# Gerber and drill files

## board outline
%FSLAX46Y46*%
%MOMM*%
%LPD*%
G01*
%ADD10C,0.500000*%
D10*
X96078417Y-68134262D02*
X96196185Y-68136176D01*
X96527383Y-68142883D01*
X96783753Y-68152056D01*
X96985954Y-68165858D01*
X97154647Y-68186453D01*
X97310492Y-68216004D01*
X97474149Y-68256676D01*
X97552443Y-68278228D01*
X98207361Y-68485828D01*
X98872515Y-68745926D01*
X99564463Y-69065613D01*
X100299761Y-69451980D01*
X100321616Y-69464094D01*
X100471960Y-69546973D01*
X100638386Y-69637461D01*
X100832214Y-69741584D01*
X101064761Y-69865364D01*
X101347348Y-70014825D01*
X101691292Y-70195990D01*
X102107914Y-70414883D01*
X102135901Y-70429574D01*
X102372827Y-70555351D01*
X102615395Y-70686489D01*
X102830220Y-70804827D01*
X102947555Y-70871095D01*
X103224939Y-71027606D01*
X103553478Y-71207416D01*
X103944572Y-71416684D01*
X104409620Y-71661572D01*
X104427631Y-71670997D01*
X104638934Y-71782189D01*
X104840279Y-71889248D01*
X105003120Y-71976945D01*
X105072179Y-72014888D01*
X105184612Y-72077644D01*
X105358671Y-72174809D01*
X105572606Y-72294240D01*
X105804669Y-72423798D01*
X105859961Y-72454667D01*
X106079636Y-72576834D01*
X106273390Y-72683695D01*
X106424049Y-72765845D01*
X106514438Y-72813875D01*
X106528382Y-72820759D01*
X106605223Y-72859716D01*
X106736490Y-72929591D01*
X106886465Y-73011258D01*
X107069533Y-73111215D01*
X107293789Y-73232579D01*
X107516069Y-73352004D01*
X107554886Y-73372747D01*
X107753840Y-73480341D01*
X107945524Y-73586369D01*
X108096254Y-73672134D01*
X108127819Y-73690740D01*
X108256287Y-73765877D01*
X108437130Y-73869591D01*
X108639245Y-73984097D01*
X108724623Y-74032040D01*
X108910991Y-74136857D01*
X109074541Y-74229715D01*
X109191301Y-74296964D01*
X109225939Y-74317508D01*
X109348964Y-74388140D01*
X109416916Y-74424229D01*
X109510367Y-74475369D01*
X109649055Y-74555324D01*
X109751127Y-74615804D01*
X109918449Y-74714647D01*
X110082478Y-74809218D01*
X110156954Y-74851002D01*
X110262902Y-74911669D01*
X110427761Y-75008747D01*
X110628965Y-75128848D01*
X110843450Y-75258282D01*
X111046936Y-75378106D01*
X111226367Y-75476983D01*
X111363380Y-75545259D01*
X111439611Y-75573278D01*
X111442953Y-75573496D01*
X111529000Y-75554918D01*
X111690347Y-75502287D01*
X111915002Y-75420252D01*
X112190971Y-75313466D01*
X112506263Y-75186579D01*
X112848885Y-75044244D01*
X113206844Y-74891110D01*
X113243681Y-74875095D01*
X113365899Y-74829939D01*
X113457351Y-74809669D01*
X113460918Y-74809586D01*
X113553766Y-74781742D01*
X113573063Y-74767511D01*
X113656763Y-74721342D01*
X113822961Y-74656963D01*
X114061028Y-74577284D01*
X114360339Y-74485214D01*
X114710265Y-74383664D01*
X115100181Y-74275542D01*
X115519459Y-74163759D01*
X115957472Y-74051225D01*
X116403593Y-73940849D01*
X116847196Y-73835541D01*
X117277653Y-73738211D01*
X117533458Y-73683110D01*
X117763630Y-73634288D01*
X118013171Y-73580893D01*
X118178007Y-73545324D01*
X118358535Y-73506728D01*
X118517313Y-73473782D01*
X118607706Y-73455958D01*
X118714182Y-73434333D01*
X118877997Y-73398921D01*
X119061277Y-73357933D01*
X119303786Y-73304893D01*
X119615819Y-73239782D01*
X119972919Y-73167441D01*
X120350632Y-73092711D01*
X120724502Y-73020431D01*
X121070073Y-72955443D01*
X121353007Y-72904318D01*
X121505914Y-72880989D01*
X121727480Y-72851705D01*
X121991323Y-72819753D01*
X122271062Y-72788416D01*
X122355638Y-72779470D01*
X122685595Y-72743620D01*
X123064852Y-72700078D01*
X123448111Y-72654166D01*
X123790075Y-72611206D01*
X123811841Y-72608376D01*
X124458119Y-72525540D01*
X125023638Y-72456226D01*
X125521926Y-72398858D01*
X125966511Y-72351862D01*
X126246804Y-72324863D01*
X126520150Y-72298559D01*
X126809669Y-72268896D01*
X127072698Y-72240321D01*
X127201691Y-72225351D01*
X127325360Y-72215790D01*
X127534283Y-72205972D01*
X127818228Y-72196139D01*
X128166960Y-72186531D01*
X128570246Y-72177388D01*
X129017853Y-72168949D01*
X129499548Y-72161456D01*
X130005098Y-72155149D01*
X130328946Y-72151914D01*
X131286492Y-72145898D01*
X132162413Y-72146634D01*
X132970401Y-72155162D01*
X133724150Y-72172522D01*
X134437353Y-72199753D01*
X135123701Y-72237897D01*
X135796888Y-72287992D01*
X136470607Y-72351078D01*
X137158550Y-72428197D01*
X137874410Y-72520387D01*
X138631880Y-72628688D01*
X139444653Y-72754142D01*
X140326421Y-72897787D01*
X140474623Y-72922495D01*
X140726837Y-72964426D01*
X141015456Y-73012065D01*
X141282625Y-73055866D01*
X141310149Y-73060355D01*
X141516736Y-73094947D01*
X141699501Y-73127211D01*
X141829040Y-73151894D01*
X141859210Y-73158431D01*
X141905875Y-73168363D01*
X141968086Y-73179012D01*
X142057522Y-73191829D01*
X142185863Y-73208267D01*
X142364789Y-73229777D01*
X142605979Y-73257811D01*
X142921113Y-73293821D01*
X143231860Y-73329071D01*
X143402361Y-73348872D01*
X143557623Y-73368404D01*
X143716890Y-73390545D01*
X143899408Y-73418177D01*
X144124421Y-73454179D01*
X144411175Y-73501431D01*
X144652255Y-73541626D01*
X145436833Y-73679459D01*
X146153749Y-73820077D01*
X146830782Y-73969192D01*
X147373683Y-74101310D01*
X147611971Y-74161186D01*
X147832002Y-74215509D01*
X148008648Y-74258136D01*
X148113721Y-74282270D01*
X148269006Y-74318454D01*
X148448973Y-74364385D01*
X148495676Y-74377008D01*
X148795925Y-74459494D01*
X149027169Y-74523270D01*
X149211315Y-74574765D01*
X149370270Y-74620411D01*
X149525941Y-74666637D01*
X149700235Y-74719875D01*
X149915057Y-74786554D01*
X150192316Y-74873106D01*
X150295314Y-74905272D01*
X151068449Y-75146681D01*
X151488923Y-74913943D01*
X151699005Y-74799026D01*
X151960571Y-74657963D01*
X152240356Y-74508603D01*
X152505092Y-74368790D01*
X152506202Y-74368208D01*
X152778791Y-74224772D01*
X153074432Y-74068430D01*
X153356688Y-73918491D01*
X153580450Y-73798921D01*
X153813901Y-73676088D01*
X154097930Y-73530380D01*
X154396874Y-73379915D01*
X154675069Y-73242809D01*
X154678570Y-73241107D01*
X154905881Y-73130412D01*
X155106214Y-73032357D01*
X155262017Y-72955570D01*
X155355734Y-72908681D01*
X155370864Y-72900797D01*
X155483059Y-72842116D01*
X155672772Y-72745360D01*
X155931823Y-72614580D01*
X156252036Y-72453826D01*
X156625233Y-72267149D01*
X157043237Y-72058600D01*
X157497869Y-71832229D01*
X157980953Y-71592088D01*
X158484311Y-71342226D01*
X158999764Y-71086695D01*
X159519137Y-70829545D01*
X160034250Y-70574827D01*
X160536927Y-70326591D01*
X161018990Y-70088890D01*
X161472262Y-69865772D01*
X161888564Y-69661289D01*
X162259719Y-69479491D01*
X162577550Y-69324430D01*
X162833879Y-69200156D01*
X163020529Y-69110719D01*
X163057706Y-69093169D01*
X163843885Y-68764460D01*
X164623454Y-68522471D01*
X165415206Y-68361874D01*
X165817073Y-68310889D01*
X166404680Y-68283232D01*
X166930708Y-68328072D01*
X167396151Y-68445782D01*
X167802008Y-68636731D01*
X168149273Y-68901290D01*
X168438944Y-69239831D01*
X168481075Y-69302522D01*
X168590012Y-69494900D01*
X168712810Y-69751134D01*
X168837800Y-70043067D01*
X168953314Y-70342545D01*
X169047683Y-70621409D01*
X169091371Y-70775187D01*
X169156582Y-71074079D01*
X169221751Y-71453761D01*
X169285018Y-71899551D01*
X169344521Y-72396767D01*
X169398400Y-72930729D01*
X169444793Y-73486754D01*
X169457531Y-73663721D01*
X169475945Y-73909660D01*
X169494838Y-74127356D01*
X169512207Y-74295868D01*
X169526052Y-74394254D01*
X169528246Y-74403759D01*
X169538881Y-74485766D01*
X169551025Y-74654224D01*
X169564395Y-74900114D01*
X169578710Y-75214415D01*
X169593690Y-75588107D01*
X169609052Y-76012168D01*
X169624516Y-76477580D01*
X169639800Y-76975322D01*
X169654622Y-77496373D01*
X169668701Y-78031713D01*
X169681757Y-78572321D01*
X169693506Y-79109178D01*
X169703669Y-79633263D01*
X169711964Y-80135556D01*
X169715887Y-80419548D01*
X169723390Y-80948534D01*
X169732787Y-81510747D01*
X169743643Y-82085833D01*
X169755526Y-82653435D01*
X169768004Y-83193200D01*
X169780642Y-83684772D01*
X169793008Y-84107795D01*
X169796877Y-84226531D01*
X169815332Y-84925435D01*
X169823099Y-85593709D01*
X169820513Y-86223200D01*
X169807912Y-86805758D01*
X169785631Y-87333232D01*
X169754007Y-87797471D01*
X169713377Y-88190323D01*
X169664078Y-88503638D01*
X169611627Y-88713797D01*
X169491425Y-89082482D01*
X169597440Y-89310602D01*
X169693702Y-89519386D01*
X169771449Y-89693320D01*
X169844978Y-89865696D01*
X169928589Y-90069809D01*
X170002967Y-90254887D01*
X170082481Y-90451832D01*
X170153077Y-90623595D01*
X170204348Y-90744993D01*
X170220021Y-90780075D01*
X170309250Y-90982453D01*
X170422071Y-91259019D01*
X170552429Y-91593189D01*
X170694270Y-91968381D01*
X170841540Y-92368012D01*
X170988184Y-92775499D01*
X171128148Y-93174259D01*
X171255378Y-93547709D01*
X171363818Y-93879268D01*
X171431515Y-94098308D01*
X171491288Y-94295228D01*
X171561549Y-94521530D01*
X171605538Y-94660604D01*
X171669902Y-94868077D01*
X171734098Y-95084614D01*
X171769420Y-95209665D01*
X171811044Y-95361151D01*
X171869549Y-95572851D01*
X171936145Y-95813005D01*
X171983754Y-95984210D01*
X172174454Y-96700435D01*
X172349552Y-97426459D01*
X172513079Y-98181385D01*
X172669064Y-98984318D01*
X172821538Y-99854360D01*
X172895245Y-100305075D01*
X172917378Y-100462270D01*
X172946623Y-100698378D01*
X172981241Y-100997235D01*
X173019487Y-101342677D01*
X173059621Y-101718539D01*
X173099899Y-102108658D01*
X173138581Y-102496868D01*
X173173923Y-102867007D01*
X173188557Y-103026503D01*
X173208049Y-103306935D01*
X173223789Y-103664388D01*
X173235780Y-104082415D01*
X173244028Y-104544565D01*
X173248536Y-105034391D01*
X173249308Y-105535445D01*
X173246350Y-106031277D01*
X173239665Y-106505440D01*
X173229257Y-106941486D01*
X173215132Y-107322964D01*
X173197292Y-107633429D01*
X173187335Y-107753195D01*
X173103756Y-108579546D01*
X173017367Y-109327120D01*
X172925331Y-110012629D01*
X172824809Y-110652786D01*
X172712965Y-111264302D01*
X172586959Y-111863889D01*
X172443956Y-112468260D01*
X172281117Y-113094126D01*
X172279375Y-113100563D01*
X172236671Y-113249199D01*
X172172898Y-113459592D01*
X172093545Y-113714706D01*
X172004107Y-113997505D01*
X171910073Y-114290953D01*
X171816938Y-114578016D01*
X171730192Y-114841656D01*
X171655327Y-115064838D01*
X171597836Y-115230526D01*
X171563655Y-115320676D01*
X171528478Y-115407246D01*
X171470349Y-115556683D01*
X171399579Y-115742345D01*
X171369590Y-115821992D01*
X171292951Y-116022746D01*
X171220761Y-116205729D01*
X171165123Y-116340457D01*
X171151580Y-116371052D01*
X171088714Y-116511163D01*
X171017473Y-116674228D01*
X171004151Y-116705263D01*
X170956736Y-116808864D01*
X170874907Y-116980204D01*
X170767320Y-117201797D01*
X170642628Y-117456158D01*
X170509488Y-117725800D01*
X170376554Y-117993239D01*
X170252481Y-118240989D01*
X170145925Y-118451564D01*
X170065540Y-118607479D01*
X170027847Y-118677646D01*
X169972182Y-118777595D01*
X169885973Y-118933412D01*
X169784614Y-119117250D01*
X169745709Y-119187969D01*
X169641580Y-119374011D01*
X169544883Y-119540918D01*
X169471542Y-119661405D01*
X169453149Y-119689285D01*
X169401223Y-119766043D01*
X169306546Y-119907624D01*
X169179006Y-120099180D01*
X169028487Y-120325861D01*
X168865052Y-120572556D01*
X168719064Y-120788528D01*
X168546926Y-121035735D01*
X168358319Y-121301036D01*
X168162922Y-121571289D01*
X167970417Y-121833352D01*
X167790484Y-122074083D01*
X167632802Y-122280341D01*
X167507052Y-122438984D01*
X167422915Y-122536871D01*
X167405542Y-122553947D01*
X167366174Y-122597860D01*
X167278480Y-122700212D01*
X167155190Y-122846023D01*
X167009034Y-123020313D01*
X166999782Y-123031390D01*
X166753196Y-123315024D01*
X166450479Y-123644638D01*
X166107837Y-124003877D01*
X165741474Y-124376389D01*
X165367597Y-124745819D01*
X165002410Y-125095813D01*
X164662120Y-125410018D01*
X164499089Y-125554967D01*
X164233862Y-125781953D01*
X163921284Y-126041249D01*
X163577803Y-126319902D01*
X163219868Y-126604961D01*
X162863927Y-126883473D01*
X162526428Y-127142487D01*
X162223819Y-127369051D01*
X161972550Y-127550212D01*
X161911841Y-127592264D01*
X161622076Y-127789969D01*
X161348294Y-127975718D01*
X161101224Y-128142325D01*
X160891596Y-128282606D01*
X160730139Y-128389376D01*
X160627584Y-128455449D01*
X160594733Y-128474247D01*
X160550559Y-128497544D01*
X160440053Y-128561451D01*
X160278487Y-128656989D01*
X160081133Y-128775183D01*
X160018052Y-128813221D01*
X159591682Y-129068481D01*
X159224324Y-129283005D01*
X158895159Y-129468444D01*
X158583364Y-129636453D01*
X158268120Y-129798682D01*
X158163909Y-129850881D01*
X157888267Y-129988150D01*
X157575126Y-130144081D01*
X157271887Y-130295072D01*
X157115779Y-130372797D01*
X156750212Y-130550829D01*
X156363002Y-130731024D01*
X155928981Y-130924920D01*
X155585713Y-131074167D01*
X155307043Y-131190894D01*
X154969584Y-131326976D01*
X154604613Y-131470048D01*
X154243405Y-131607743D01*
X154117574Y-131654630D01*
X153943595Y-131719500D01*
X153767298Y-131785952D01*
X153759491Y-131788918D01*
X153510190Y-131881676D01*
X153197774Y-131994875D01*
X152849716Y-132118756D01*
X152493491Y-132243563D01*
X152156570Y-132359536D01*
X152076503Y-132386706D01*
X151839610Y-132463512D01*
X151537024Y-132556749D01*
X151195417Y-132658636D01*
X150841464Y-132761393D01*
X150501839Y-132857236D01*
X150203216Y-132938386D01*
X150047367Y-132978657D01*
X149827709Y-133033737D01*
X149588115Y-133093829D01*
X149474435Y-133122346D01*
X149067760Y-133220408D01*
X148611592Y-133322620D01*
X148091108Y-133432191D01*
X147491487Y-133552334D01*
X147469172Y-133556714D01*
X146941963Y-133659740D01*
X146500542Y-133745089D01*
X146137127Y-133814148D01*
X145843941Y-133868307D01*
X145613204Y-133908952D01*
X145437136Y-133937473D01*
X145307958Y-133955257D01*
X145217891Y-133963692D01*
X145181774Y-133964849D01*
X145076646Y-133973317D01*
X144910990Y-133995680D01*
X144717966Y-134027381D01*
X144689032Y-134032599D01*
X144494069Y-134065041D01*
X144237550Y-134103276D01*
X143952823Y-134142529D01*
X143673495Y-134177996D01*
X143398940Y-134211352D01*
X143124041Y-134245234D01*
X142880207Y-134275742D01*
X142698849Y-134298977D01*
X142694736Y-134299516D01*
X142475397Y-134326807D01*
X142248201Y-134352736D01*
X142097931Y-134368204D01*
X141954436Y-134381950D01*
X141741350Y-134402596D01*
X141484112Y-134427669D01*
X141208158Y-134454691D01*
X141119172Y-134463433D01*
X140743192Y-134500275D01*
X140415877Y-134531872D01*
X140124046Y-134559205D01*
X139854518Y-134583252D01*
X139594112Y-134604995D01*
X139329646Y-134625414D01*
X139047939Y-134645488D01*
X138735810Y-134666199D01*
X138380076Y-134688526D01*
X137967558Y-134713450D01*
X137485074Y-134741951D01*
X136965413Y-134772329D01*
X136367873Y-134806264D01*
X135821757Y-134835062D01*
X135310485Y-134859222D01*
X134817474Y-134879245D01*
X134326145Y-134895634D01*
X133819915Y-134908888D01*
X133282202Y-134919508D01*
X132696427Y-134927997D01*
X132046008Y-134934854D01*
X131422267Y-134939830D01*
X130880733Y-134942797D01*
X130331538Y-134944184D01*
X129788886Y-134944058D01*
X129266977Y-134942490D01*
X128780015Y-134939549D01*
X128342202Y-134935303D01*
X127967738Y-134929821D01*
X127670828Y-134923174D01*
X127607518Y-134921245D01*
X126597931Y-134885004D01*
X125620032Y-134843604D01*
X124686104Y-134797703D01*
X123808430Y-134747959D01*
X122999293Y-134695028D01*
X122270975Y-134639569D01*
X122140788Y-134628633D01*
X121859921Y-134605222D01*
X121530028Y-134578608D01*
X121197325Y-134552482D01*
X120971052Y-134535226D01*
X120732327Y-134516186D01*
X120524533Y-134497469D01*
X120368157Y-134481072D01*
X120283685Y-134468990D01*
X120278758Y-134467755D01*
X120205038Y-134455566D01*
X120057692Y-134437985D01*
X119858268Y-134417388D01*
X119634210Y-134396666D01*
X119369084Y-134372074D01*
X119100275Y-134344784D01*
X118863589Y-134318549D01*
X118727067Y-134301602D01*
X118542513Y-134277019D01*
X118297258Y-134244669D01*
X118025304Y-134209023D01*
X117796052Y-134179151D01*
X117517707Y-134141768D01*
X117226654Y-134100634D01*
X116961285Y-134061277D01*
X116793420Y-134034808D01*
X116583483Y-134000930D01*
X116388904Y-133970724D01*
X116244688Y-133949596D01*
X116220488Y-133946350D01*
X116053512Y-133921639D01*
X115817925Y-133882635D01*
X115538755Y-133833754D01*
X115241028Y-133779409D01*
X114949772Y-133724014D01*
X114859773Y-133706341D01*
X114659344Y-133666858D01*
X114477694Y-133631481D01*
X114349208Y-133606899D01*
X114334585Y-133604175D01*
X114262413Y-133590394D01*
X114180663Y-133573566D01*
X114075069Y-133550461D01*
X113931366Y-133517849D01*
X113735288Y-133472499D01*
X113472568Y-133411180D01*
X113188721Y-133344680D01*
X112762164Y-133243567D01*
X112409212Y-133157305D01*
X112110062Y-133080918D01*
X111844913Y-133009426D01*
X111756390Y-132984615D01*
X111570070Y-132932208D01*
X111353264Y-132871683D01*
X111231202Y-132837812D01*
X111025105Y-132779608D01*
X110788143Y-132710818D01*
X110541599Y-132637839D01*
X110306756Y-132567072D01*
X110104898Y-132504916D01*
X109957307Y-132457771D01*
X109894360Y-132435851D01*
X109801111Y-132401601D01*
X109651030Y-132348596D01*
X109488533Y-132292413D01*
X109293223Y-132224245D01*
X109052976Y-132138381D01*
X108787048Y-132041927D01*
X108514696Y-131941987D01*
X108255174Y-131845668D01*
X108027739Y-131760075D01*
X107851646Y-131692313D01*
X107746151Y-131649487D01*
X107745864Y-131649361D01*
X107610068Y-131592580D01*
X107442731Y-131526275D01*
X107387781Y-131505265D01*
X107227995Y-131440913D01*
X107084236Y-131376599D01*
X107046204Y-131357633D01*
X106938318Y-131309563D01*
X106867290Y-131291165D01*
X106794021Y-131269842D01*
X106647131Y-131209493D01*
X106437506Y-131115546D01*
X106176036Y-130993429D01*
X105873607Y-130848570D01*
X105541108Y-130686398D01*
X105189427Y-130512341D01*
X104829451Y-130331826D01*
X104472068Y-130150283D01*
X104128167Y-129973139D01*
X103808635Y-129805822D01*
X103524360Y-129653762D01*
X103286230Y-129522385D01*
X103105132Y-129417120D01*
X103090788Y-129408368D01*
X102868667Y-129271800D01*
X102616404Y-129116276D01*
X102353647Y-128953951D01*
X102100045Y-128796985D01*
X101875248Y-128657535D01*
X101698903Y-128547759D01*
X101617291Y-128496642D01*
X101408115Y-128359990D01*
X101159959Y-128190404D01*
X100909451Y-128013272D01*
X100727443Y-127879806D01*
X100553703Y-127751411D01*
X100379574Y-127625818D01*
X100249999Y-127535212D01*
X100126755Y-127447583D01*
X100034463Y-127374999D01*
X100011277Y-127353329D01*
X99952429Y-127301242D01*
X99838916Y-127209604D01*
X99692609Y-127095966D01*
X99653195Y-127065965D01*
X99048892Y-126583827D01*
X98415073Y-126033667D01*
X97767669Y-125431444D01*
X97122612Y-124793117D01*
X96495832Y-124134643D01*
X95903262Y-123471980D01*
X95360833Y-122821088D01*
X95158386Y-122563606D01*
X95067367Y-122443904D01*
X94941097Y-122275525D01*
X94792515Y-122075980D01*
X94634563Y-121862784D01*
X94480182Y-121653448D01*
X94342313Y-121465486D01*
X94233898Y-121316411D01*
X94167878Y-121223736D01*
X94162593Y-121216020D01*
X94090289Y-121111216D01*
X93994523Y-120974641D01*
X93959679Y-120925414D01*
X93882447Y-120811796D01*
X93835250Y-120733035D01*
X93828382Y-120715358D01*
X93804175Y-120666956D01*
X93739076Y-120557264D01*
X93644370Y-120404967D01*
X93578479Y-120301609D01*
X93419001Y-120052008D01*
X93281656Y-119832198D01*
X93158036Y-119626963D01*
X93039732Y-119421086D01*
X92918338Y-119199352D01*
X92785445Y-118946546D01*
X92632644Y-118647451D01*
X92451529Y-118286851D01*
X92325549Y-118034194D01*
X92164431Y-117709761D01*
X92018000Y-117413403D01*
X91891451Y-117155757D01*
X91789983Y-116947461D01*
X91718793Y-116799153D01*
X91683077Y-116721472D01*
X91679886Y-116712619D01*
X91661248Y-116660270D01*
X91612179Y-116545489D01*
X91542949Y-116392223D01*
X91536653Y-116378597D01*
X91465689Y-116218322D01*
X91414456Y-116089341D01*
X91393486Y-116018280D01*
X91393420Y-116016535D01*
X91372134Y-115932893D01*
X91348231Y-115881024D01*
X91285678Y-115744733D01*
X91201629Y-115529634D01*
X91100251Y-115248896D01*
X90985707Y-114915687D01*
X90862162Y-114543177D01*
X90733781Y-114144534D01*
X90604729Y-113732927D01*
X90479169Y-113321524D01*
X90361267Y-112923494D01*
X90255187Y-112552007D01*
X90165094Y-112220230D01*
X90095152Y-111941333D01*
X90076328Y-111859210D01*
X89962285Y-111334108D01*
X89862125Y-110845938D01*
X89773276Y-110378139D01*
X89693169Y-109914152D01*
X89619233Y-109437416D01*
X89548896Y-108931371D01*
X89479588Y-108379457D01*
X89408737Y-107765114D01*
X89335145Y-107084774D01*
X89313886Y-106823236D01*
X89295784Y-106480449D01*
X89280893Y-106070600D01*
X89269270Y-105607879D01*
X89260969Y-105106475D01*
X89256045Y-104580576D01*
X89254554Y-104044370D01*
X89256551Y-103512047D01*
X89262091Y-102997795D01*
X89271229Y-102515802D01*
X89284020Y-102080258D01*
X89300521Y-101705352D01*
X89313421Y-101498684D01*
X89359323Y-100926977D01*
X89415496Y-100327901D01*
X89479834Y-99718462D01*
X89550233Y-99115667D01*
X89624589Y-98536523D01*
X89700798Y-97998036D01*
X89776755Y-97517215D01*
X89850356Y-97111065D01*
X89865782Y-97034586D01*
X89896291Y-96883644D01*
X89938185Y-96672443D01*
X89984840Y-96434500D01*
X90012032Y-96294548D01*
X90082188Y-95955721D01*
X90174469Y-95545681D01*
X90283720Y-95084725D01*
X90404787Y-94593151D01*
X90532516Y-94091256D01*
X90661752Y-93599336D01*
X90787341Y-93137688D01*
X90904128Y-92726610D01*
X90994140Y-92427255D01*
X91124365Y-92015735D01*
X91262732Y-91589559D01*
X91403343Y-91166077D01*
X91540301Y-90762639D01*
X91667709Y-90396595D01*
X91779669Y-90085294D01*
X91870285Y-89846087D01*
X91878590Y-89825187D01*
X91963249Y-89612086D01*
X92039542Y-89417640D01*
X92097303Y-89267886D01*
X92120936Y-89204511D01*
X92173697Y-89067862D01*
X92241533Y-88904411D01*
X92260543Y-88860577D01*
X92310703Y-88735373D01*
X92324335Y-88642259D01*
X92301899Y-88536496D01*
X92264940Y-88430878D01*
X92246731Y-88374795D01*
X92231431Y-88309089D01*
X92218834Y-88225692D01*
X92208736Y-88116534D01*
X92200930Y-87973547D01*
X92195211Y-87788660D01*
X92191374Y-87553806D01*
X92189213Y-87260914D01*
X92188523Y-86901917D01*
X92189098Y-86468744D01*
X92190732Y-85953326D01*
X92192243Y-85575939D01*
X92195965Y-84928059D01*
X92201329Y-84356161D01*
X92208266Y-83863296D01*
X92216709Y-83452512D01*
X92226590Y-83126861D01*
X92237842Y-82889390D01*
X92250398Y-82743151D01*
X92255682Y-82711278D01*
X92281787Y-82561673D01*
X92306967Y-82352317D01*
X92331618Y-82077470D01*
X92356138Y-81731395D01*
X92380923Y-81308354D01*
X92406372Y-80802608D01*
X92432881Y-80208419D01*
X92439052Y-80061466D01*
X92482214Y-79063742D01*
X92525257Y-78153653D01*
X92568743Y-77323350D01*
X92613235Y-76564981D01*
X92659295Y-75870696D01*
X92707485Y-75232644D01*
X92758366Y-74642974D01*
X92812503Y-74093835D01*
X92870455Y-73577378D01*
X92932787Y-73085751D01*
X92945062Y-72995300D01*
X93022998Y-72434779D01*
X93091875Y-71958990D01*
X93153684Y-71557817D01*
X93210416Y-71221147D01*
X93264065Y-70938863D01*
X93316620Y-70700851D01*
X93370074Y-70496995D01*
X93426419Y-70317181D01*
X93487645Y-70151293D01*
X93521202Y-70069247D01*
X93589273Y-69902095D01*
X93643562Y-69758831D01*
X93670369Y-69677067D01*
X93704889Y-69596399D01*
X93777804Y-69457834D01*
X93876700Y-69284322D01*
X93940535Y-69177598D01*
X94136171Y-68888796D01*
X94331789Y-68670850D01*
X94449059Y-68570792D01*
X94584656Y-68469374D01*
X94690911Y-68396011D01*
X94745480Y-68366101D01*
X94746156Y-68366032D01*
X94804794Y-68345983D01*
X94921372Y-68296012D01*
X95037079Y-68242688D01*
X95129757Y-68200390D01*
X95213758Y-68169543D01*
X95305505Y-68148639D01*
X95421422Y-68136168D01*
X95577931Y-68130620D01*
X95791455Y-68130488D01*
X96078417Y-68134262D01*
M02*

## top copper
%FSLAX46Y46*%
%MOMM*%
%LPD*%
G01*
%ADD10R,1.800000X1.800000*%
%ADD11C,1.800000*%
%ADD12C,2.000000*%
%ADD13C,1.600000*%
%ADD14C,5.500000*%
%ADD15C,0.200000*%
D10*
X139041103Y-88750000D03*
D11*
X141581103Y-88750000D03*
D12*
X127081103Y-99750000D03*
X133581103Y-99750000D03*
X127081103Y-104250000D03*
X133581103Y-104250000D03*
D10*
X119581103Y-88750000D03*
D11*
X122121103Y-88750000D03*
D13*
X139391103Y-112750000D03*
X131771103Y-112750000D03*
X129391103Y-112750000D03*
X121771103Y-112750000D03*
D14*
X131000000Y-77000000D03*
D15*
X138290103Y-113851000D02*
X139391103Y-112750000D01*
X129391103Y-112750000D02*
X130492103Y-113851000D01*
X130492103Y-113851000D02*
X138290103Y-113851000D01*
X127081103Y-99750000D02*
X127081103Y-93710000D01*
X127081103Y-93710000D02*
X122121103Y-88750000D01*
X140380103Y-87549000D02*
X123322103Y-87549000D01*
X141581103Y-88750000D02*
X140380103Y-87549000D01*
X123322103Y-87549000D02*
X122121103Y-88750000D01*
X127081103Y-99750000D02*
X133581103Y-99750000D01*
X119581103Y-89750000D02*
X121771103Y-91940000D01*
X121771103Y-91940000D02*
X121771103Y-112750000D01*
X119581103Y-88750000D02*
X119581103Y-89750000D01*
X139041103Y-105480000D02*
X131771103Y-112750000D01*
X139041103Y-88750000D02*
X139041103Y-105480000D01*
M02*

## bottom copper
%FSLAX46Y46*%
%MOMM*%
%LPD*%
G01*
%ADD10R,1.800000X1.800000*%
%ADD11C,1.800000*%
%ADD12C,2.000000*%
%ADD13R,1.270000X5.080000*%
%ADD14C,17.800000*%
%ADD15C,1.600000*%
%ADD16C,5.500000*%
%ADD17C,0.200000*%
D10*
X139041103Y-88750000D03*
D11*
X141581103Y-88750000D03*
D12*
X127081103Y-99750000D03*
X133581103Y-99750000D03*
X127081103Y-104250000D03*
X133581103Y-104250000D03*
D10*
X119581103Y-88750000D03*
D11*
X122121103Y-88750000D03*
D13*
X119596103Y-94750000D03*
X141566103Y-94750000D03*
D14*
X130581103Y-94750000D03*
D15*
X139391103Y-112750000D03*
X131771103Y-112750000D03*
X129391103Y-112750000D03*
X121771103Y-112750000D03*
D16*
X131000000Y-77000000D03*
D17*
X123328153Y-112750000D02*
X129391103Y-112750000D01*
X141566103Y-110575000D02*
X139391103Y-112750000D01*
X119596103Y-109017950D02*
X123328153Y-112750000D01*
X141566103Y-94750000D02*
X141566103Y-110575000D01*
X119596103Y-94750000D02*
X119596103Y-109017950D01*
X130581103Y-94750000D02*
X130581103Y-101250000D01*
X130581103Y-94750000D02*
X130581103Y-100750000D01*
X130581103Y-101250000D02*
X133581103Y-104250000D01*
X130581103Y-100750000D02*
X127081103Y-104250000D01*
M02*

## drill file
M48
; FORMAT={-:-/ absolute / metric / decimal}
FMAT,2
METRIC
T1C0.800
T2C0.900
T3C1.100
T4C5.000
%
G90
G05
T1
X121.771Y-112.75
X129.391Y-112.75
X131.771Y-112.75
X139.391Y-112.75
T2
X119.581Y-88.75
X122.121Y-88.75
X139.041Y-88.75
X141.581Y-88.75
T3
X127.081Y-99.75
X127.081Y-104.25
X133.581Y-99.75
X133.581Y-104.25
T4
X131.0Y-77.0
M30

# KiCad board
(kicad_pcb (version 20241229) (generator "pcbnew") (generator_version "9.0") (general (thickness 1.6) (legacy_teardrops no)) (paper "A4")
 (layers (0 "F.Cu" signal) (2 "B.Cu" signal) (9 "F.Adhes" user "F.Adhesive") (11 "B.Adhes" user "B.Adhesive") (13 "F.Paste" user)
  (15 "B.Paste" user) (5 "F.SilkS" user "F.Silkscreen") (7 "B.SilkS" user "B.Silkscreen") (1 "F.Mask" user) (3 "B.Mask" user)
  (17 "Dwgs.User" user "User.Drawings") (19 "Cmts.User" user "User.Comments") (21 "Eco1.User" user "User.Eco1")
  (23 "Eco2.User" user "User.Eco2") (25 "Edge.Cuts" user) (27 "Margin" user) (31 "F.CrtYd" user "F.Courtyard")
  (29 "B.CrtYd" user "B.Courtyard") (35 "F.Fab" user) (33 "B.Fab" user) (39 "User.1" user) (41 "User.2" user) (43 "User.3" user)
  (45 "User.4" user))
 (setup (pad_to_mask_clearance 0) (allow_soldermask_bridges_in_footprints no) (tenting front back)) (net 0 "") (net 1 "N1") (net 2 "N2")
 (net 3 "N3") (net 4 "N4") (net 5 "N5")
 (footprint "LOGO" (layer "F.Cu") (at 100 77 10)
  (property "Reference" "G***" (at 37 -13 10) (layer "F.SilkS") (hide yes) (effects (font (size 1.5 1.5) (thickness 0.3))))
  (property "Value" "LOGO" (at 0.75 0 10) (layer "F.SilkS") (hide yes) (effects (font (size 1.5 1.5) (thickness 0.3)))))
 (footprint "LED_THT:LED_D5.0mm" (layer "F.Cu") (at 139.041103 88.75)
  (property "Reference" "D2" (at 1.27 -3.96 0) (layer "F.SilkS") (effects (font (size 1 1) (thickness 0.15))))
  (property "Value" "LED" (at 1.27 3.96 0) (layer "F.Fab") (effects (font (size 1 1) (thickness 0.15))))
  (pad "1" thru_hole rect (at 0 0) (size 1.8 1.8) (drill 0.9) (layers "*.Cu" "*.Mask") (remove_unused_layers no) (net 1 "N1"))
  (pad "2" thru_hole circle (at 2.54 0) (size 1.8 1.8) (drill 0.9) (layers "*.Cu" "*.Mask") (remove_unused_layers no) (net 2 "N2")))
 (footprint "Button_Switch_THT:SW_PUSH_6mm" (layer "F.Cu") (at 127.081103 99.75)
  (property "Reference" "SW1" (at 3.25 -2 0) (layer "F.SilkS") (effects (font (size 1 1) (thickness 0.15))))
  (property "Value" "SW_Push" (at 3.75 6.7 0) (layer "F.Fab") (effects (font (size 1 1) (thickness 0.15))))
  (pad "1" thru_hole circle (at 0 0 90) (size 2 2) (drill 1.1) (layers "*.Cu" "*.Mask") (remove_unused_layers no) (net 2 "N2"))
  (pad "1" thru_hole circle (at 6.5 0 90) (size 2 2) (drill 1.1) (layers "*.Cu" "*.Mask") (remove_unused_layers no) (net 2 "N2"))
  (pad "2" thru_hole circle (at 0 4.5 90) (size 2 2) (drill 1.1) (layers "*.Cu" "*.Mask") (remove_unused_layers no) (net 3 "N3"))
  (pad "2" thru_hole circle (at 6.5 4.5 90) (size 2 2) (drill 1.1) (layers "*.Cu" "*.Mask") (remove_unused_layers no) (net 3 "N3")))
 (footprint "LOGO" (layer "F.Cu") (at 132 102)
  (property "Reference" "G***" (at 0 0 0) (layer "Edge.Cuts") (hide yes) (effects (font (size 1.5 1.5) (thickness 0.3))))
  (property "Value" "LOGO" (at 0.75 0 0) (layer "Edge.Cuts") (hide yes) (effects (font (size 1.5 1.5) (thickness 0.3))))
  (fp_poly
   (pts (xy -35.921583 -33.865738) (xy -35.803815 -33.863824) (xy -35.472617 -33.857117) (xy -35.216247 -33.847944)
    (xy -35.014046 -33.834142) (xy -34.845353 -33.813547) (xy -34.689508 -33.783996) (xy -34.525851 -33.743324) (xy -34.447557 -33.721772)
    (xy -33.792639 -33.514172) (xy -33.127485 -33.254074) (xy -32.435537 -32.934387) (xy -31.700239 -32.54802) (xy -31.678384 -32.535906)
    (xy -31.52804 -32.453027) (xy -31.361614 -32.362539) (xy -31.167786 -32.258416) (xy -30.935239 -32.134636) (xy -30.652652 -31.985175)
    (xy -30.308708 -31.80401) (xy -29.892086 -31.585117) (xy -29.864099 -31.570426) (xy -29.627173 -31.444649) (xy -29.384605 -31.313511)
    (xy -29.16978 -31.195173) (xy -29.052445 -31.128905) (xy -28.775061 -30.972394) (xy -28.446522 -30.792584) (xy -28.055428 -30.583316)
    (xy -27.59038 -30.338428) (xy -27.572369 -30.329003) (xy -27.361066 -30.217811) (xy -27.159721 -30.110752) (xy -26.99688 -30.023055)
    (xy -26.927821 -29.985112) (xy -26.815388 -29.922356) (xy -26.641329 -29.825191) (xy -26.427394 -29.70576) (xy -26.195331 -29.576202)
    (xy -26.140039 -29.545333) (xy -25.920364 -29.423166) (xy -25.72661 -29.316305) (xy -25.575951 -29.234155) (xy -25.485562 -29.186125)
    (xy -25.471618 -29.179241) (xy -25.394777 -29.140284) (xy -25.26351 -29.070409) (xy -25.113535 -28.988742) (xy -24.930467 -28.888785)
    (xy -24.706211 -28.767421) (xy -24.483931 -28.647996) (xy -24.445114 -28.627253) (xy -24.24616 -28.519659) (xy -24.054476 -28.413631)
    (xy -23.903746 -28.327866) (xy -23.872181 -28.30926) (xy -23.743713 -28.234123) (xy -23.56287 -28.130409) (xy -23.360755 -28.015903)
    (xy -23.275377 -27.96796) (xy -23.089009 -27.863143) (xy -22.925459 -27.770285) (xy -22.808699 -27.703036) (xy -22.774061 -27.682492)
    (xy -22.651036 -27.61186) (xy -22.583084 -27.575771) (xy -22.489633 -27.524631) (xy -22.350945 -27.444676) (xy -22.248873 -27.384196)
    (xy -22.081551 -27.285353) (xy -21.917522 -27.190782) (xy -21.843046 -27.148998) (xy -21.737098 -27.088331) (xy -21.572239 -26.991253)
    (xy -21.371035 -26.871152) (xy -21.15655 -26.741718) (xy -20.953064 -26.621894) (xy -20.773633 -26.523017) (xy -20.63662 -26.454741)
    (xy -20.560389 -26.426722) (xy -20.557047 -26.426504) (xy -20.471 -26.445082) (xy -20.309653 -26.497713) (xy -20.084998 -26.579748)
    (xy -19.809029 -26.686534) (xy -19.493737 -26.813421) (xy -19.151115 -26.955756) (xy -18.793156 -27.10889) (xy -18.756319 -27.124905)
    (xy -18.634101 -27.170061) (xy -18.542649 -27.190331) (xy -18.539082 -27.190414) (xy -18.446234 -27.218258) (xy -18.426937 -27.232489)
    (xy -18.343237 -27.278658) (xy -18.177039 -27.343037) (xy -17.938972 -27.422716) (xy -17.639661 -27.514786) (xy -17.289735 -27.616336)
    (xy -16.899819 -27.724458) (xy -16.480541 -27.836241) (xy -16.042528 -27.948775) (xy -15.596407 -28.059151) (xy -15.152804 -28.164459)
    (xy -14.722347 -28.261789) (xy -14.466542 -28.31689) (xy -14.23637 -28.365712) (xy -13.986829 -28.419107) (xy -13.821993 -28.454676)
    (xy -13.641465 -28.493272) (xy -13.482687 -28.526218) (xy -13.392294 -28.544042) (xy -13.285818 -28.565667) (xy -13.122003 -28.601079)
    (xy -12.938723 -28.642067) (xy -12.696214 -28.695107) (xy -12.384181 -28.760218) (xy -12.027081 -28.832559) (xy -11.649368 -28.907289)
    (xy -11.275498 -28.979569) (xy -10.929927 -29.044557) (xy -10.646993 -29.095682) (xy -10.494086 -29.119011) (xy -10.27252 -29.148295)
    (xy -10.008677 -29.180247) (xy -9.728938 -29.211584) (xy -9.644362 -29.22053) (xy -9.314405 -29.25638) (xy -8.935148 -29.299922)
    (xy -8.551889 -29.345834) (xy -8.209925 -29.388794) (xy -8.188159 -29.391624) (xy -7.541881 -29.47446) (xy -6.976362 -29.543774)
    (xy -6.478074 -29.601142) (xy -6.033489 -29.648138) (xy -5.753196 -29.675137) (xy -5.47985 -29.701441) (xy -5.190331 -29.731104)
    (xy -4.927302 -29.759679) (xy -4.798309 -29.774649) (xy -4.67464 -29.78421) (xy -4.465717 -29.794028) (xy -4.181772 -29.803861)
    (xy -3.83304 -29.813469) (xy -3.429754 -29.822612) (xy -2.982147 -29.831051) (xy -2.500452 -29.838544) (xy -1.994902 -29.844851)
    (xy -1.671054 -29.848086) (xy -0.713508 -29.854102) (xy 0.162413 -29.853366) (xy 0.970401 -29.844838) (xy 1.72415 -29.827478)
    (xy 2.437353 -29.800247) (xy 3.123701 -29.762103) (xy 3.796888 -29.712008) (xy 4.470607 -29.648922) (xy 5.15855 -29.571803)
    (xy 5.87441 -29.479613) (xy 6.63188 -29.371312) (xy 7.444653 -29.245858) (xy 8.326421 -29.102213) (xy 8.474623 -29.077505)
    (xy 8.726837 -29.035574) (xy 9.015456 -28.987935) (xy 9.282625 -28.944134) (xy 9.310149 -28.939645) (xy 9.516736 -28.905053)
    (xy 9.699501 -28.872789) (xy 9.82904 -28.848106) (xy 9.85921 -28.841569) (xy 9.905875 -28.831637) (xy 9.968086 -28.820988)
    (xy 10.057522 -28.808171) (xy 10.185863 -28.791733) (xy 10.364789 -28.770223) (xy 10.605979 -28.742189) (xy 10.921113 -28.706179)
    (xy 11.23186 -28.670929) (xy 11.402361 -28.651128) (xy 11.557623 -28.631596) (xy 11.71689 -28.609455) (xy 11.899408 -28.581823)
    (xy 12.124421 -28.545821) (xy 12.411175 -28.498569) (xy 12.652255 -28.458374) (xy 13.436833 -28.320541) (xy 14.153749 -28.179923)
    (xy 14.830782 -28.030808) (xy 15.373683 -27.89869) (xy 15.611971 -27.838814) (xy 15.832002 -27.784491) (xy 16.008648 -27.741864)
    (xy 16.113721 -27.71773) (xy 16.269006 -27.681546) (xy 16.448973 -27.635615) (xy 16.495676 -27.622992) (xy 16.795925 -27.540506)
    (xy 17.027169 -27.47673) (xy 17.211315 -27.425235) (xy 17.37027 -27.379589) (xy 17.525941 -27.333363) (xy 17.700235 -27.280125)
    (xy 17.915057 -27.213446) (xy 18.192316 -27.126894) (xy 18.295314 -27.094728) (xy 19.068449 -26.853319) (xy 19.488923 -27.086057)
    (xy 19.699005 -27.200974) (xy 19.960571 -27.342037) (xy 20.240356 -27.491397) (xy 20.505092 -27.63121) (xy 20.506202 -27.631792)
    (xy 20.778791 -27.775228) (xy 21.074432 -27.93157) (xy 21.356688 -28.081509) (xy 21.58045 -28.201079) (xy 21.813901 -28.323912)
    (xy 22.09793 -28.46962) (xy 22.396874 -28.620085) (xy 22.675069 -28.757191) (xy 22.67857 -28.758893) (xy 22.905881 -28.869588)
    (xy 23.106214 -28.967643) (xy 23.262017 -29.04443) (xy 23.355734 -29.091319) (xy 23.370864 -29.099203) (xy 23.483059 -29.157884)
    (xy 23.672772 -29.25464) (xy 23.931823 -29.38542) (xy 24.252036 -29.546174) (xy 24.625233 -29.732851) (xy 25.043237 -29.9414)
    (xy 25.497869 -30.167771) (xy 25.980953 -30.407912) (xy 26.484311 -30.657774) (xy 26.999764 -30.913305) (xy 27.519137 -31.170455)
    (xy 28.03425 -31.425173) (xy 28.536927 -31.673409) (xy 29.01899 -31.91111) (xy 29.472262 -32.134228) (xy 29.888564 -32.338711)
    (xy 30.259719 -32.520509) (xy 30.57755 -32.67557) (xy 30.833879 -32.799844) (xy 31.020529 -32.889281) (xy 31.057706 -32.906831)
    (xy 31.843885 -33.23554) (xy 32.623454 -33.477529) (xy 33.415206 -33.638126) (xy 33.817073 -33.689111) (xy 34.40468 -33.716768)
    (xy 34.930708 -33.671928) (xy 35.396151 -33.554218) (xy 35.802008 -33.363269) (xy 36.149273 -33.09871) (xy 36.438944 -32.760169)
    (xy 36.481075 -32.697478) (xy 36.590012 -32.5051) (xy 36.71281 -32.248866) (xy 36.8378 -31.956933) (xy 36.953314 -31.657455)
    (xy 37.047683 -31.378591) (xy 37.091371 -31.224813) (xy 37.156582 -30.925921) (xy 37.221751 -30.546239) (xy 37.285018 -30.100449)
    (xy 37.344521 -29.603233) (xy 37.3984 -29.069271) (xy 37.444793 -28.513246) (xy 37.457531 -28.336279) (xy 37.475945 -28.09034)
    (xy 37.494838 -27.872644) (xy 37.512207 -27.704132) (xy 37.526052 -27.605746) (xy 37.528246 -27.596241) (xy 37.538881 -27.514234)
    (xy 37.551025 -27.345776) (xy 37.564395 -27.099886) (xy 37.57871 -26.785585) (xy 37.59369 -26.411893) (xy 37.609052 -25.987832)
    (xy 37.624516 -25.52242) (xy 37.6398 -25.024678) (xy 37.654622 -24.503627) (xy 37.668701 -23.968287) (xy 37.681757 -23.427679)
    (xy 37.693506 -22.890822) (xy 37.703669 -22.366737) (xy 37.711964 -21.864444) (xy 37.715887 -21.580452) (xy 37.72339 -21.051466)
    (xy 37.732787 -20.489253) (xy 37.743643 -19.914167) (xy 37.755526 -19.346565) (xy 37.768004 -18.8068) (xy 37.780642 -18.315228)
    (xy 37.793008 -17.892205) (xy 37.796877 -17.773469) (xy 37.815332 -17.074565) (xy 37.823099 -16.406291) (xy 37.820513 -15.7768)
    (xy 37.807912 -15.194242) (xy 37.785631 -14.666768) (xy 37.754007 -14.202529) (xy 37.713377 -13.809677) (xy 37.664078 -13.496362)
    (xy 37.611627 -13.286203) (xy 37.491425 -12.917518) (xy 37.59744 -12.689398) (xy 37.693702 -12.480614) (xy 37.771449 -12.30668)
    (xy 37.844978 -12.134304) (xy 37.928589 -11.930191) (xy 38.002967 -11.745113) (xy 38.082481 -11.548168) (xy 38.153077 -11.376405)
    (xy 38.204348 -11.255007) (xy 38.220021 -11.219925) (xy 38.30925 -11.017547) (xy 38.422071 -10.740981) (xy 38.552429 -10.406811)
    (xy 38.69427 -10.031619) (xy 38.84154 -9.631988) (xy 38.988184 -9.224501) (xy 39.128148 -8.825741) (xy 39.255378 -8.452291)
    (xy 39.363818 -8.120732) (xy 39.431515 -7.901692) (xy 39.491288 -7.704772) (xy 39.561549 -7.47847) (xy 39.605538 -7.339396)
    (xy 39.669902 -7.131923) (xy 39.734098 -6.915386) (xy 39.76942 -6.790335) (xy 39.811044 -6.638849) (xy 39.869549 -6.427149)
    (xy 39.936145 -6.186995) (xy 39.983754 -6.01579) (xy 40.174454 -5.299565) (xy 40.349552 -4.573541) (xy 40.513079 -3.818615)
    (xy 40.669064 -3.015682) (xy 40.821538 -2.14564) (xy 40.895245 -1.694925) (xy 40.917378 -1.53773) (xy 40.946623 -1.301622)
    (xy 40.981241 -1.002765) (xy 41.019487 -0.657323) (xy 41.059621 -0.281461) (xy 41.099899 0.108658) (xy 41.138581 0.496868)
    (xy 41.173923 0.867007) (xy 41.188557 1.026503) (xy 41.208049 1.306935) (xy 41.223789 1.664388) (xy 41.23578 2.082415)
    (xy 41.244028 2.544565) (xy 41.248536 3.034391) (xy 41.249308 3.535445) (xy 41.24635 4.031277) (xy 41.239665 4.50544)
    (xy 41.229257 4.941486) (xy 41.215132 5.322964) (xy 41.197292 5.633429) (xy 41.187335 5.753195) (xy 41.103756 6.579546)
    (xy 41.017367 7.32712) (xy 40.925331 8.012629) (xy 40.824809 8.652786) (xy 40.712965 9.264302) (xy 40.586959 9.863889)
    (xy 40.443956 10.46826) (xy 40.281117 11.094126) (xy 40.279375 11.100563) (xy 40.236671 11.249199) (xy 40.172898 11.459592)
    (xy 40.093545 11.714706) (xy 40.004107 11.997505) (xy 39.910073 12.290953) (xy 39.816938 12.578016) (xy 39.730192 12.841656)
    (xy 39.655327 13.064838) (xy 39.597836 13.230526) (xy 39.563655 13.320676) (xy 39.528478 13.407246) (xy 39.470349 13.556683)
    (xy 39.399579 13.742345) (xy 39.36959 13.821992) (xy 39.292951 14.022746) (xy 39.220761 14.205729) (xy 39.165123 14.340457)
    (xy 39.15158 14.371052) (xy 39.088714 14.511163) (xy 39.017473 14.674228) (xy 39.004151 14.705263) (xy 38.956736 14.808864)
    (xy 38.874907 14.980204) (xy 38.76732 15.201797) (xy 38.642628 15.456158) (xy 38.509488 15.7258) (xy 38.376554 15.993239)
    (xy 38.252481 16.240989) (xy 38.145925 16.451564) (xy 38.06554 16.607479) (xy 38.027847 16.677646) (xy 37.972182 16.777595)
    (xy 37.885973 16.933412) (xy 37.784614 17.11725) (xy 37.745709 17.187969) (xy 37.64158 17.374011) (xy 37.544883 17.540918)
    (xy 37.471542 17.661405) (xy 37.453149 17.689285) (xy 37.401223 17.766043) (xy 37.306546 17.907624) (xy 37.179006 18.09918)
    (xy 37.028487 18.325861) (xy 36.865052 18.572556) (xy 36.719064 18.788528) (xy 36.546926 19.035735) (xy 36.358319 19.301036)
    (xy 36.162922 19.571289) (xy 35.970417 19.833352) (xy 35.790484 20.074083) (xy 35.632802 20.280341) (xy 35.507052 20.438984)
    (xy 35.422915 20.536871) (xy 35.405542 20.553947) (xy 35.366174 20.59786) (xy 35.27848 20.700212) (xy 35.15519 20.846023)
    (xy 35.009034 21.020313) (xy 34.999782 21.03139) (xy 34.753196 21.315024) (xy 34.450479 21.644638) (xy 34.107837 22.003877)
    (xy 33.741474 22.376389) (xy 33.367597 22.745819) (xy 33.00241 23.095813) (xy 32.66212 23.410018) (xy 32.499089 23.554967)
    (xy 32.233862 23.781953) (xy 31.921284 24.041249) (xy 31.577803 24.319902) (xy 31.219868 24.604961) (xy 30.863927 24.883473)
    (xy 30.526428 25.142487) (xy 30.223819 25.369051) (xy 29.97255 25.550212) (xy 29.911841 25.592264) (xy 29.622076 25.789969)
    (xy 29.348294 25.975718) (xy 29.101224 26.142325) (xy 28.891596 26.282606) (xy 28.730139 26.389376) (xy 28.627584 26.455449)
    (xy 28.594733 26.474247) (xy 28.550559 26.497544) (xy 28.440053 26.561451) (xy 28.278487 26.656989) (xy 28.081133 26.775183)
    (xy 28.018052 26.813221) (xy 27.591682 27.068481) (xy 27.224324 27.283005) (xy 26.895159 27.468444) (xy 26.583364 27.636453)
    (xy 26.26812 27.798682) (xy 26.163909 27.850881) (xy 25.888267 27.98815) (xy 25.575126 28.144081) (xy 25.271887 28.295072)
    (xy 25.115779 28.372797) (xy 24.750212 28.550829) (xy 24.363002 28.731024) (xy 23.928981 28.92492) (xy 23.585713 29.074167)
    (xy 23.307043 29.190894) (xy 22.969584 29.326976) (xy 22.604613 29.470048) (xy 22.243405 29.607743) (xy 22.117574 29.65463)
    (xy 21.943595 29.7195) (xy 21.767298 29.785952) (xy 21.759491 29.788918) (xy 21.51019 29.881676) (xy 21.197774 29.994875)
    (xy 20.849716 30.118756) (xy 20.493491 30.243563) (xy 20.15657 30.359536) (xy 20.076503 30.386706) (xy 19.83961 30.463512)
    (xy 19.537024 30.556749) (xy 19.195417 30.658636) (xy 18.841464 30.761393) (xy 18.501839 30.857236) (xy 18.203216 30.938386)
    (xy 18.047367 30.978657) (xy 17.827709 31.033737) (xy 17.588115 31.093829) (xy 17.474435 31.122346) (xy 17.06776 31.220408)
    (xy 16.611592 31.32262) (xy 16.091108 31.432191) (xy 15.491487 31.552334) (xy 15.469172 31.556714) (xy 14.941963 31.65974)
    (xy 14.500542 31.745089) (xy 14.137127 31.814148) (xy 13.843941 31.868307) (xy 13.613204 31.908952) (xy 13.437136 31.937473)
    (xy 13.307958 31.955257) (xy 13.217891 31.963692) (xy 13.181774 31.964849) (xy 13.076646 31.973317) (xy 12.91099 31.99568)
    (xy 12.717966 32.027381) (xy 12.689032 32.032599) (xy 12.494069 32.065041) (xy 12.23755 32.103276) (xy 11.952823 32.142529)
    (xy 11.673495 32.177996) (xy 11.39894 32.211352) (xy 11.124041 32.245234) (xy 10.880207 32.275742) (xy 10.698849 32.298977)
    (xy 10.694736 32.299516) (xy 10.475397 32.326807) (xy 10.248201 32.352736) (xy 10.097931 32.368204) (xy 9.954436 32.38195)
    (xy 9.74135 32.402596) (xy 9.484112 32.427669) (xy 9.208158 32.454691) (xy 9.119172 32.463433) (xy 8.743192 32.500275)
    (xy 8.415877 32.531872) (xy 8.124046 32.559205) (xy 7.854518 32.583252) (xy 7.594112 32.604995) (xy 7.329646 32.625414)
    (xy 7.047939 32.645488) (xy 6.73581 32.666199) (xy 6.380076 32.688526) (xy 5.967558 32.71345) (xy 5.485074 32.741951)
    (xy 4.965413 32.772329) (xy 4.367873 32.806264) (xy 3.821757 32.835062) (xy 3.310485 32.859222) (xy 2.817474 32.879245)
    (xy 2.326145 32.895634) (xy 1.819915 32.908888) (xy 1.282202 32.919508) (xy 0.696427 32.927997) (xy 0.046008 32.934854)
    (xy -0.577733 32.93983) (xy -1.119267 32.942797) (xy -1.668462 32.944184) (xy -2.211114 32.944058) (xy -2.733023 32.94249)
    (xy -3.219985 32.939549) (xy -3.657798 32.935303) (xy -4.032262 32.929821) (xy -4.329172 32.923174) (xy -4.392482 32.921245)
    (xy -5.402069 32.885004) (xy -6.379968 32.843604) (xy -7.313896 32.797703) (xy -8.19157 32.747959) (xy -9.000707 32.695028)
    (xy -9.729025 32.639569) (xy -9.859212 32.628633) (xy -10.140079 32.605222) (xy -10.469972 32.578608) (xy -10.802675 32.552482)
    (xy -11.028948 32.535226) (xy -11.267673 32.516186) (xy -11.475467 32.497469) (xy -11.631843 32.481072) (xy -11.716315 32.46899)
    (xy -11.721242 32.467755) (xy -11.794962 32.455566) (xy -11.942308 32.437985) (xy -12.141732 32.417388) (xy -12.36579 32.396666)
    (xy -12.630916 32.372074) (xy -12.899725 32.344784) (xy -13.136411 32.318549) (xy -13.272933 32.301602) (xy -13.457487 32.277019)
    (xy -13.702742 32.244669) (xy -13.974696 32.209023) (xy -14.203948 32.179151) (xy -14.482293 32.141768) (xy -14.773346 32.100634)
    (xy -15.038715 32.061277) (xy -15.20658 32.034808) (xy -15.416517 32.00093) (xy -15.611096 31.970724) (xy -15.755312 31.949596)
    (xy -15.779512 31.94635) (xy -15.946488 31.921639) (xy -16.182075 31.882635) (xy -16.461245 31.833754) (xy -16.758972 31.779409)
    (xy -17.050228 31.724014) (xy -17.140227 31.706341) (xy -17.340656 31.666858) (xy -17.522306 31.631481) (xy -17.650792 31.606899)
    (xy -17.665415 31.604175) (xy -17.737587 31.590394) (xy -17.819337 31.573566) (xy -17.924931 31.550461) (xy -18.068634 31.517849)
    (xy -18.264712 31.472499) (xy -18.527432 31.41118) (xy -18.811279 31.34468) (xy -19.237836 31.243567) (xy -19.590788 31.157305)
    (xy -19.889938 31.080918) (xy -20.155087 31.009426) (xy -20.24361 30.984615) (xy -20.42993 30.932208) (xy -20.646736 30.871683)
    (xy -20.768798 30.837812) (xy -20.974895 30.779608) (xy -21.211857 30.710818) (xy -21.458401 30.637839) (xy -21.693244 30.567072)
    (xy -21.895102 30.504916) (xy -22.042693 30.457771) (xy -22.10564 30.435851) (xy -22.198889 30.401601) (xy -22.34897 30.348596)
    (xy -22.511467 30.292413) (xy -22.706777 30.224245) (xy -22.947024 30.138381) (xy -23.212952 30.041927) (xy -23.485304 29.941987)
    (xy -23.744826 29.845668) (xy -23.972261 29.760075) (xy -24.148354 29.692313) (xy -24.253849 29.649487) (xy -24.254136 29.649361)
    (xy -24.389932 29.59258) (xy -24.557269 29.526275) (xy -24.612219 29.505265) (xy -24.772005 29.440913) (xy -24.915764 29.376599)
    (xy -24.953796 29.357633) (xy -25.061682 29.309563) (xy -25.13271 29.291165) (xy -25.205979 29.269842) (xy -25.352869 29.209493)
    (xy -25.562494 29.115546) (xy -25.823964 28.993429) (xy -26.126393 28.84857) (xy -26.458892 28.686398) (xy -26.810573 28.512341)
    (xy -27.170549 28.331826) (xy -27.527932 28.150283) (xy -27.871833 27.973139) (xy -28.191365 27.805822) (xy -28.47564 27.653762)
    (xy -28.71377 27.522385) (xy -28.894868 27.41712) (xy -28.909212 27.408368) (xy -29.131333 27.2718) (xy -29.383596 27.116276)
    (xy -29.646353 26.953951) (xy -29.899955 26.796985) (xy -30.124752 26.657535) (xy -30.301097 26.547759) (xy -30.382709 26.496642)
    (xy -30.591885 26.35999) (xy -30.840041 26.190404) (xy -31.090549 26.013272) (xy -31.272557 25.879806) (xy -31.446297 25.751411)
    (xy -31.620426 25.625818) (xy -31.750001 25.535212) (xy -31.873245 25.447583) (xy -31.965537 25.374999) (xy -31.988723 25.353329)
    (xy -32.047571 25.301242) (xy -32.161084 25.209604) (xy -32.307391 25.095966) (xy -32.346805 25.065965) (xy -32.951108 24.583827)
    (xy -33.584927 24.033667) (xy -34.232331 23.431444) (xy -34.877388 22.793117) (xy -35.504168 22.134643) (xy -36.096738 21.47198)
    (xy -36.639167 20.821088) (xy -36.841614 20.563606) (xy -36.932633 20.443904) (xy -37.058903 20.275525) (xy -37.207485 20.07598)
    (xy -37.365437 19.862784) (xy -37.519818 19.653448) (xy -37.657687 19.465486) (xy -37.766102 19.316411) (xy -37.832122 19.223736)
    (xy -37.837407 19.21602) (xy -37.909711 19.111216) (xy -38.005477 18.974641) (xy -38.040321 18.925414) (xy -38.117553 18.811796)
    (xy -38.16475 18.733035) (xy -38.171618 18.715358) (xy -38.195825 18.666956) (xy -38.260924 18.557264) (xy -38.35563 18.404967)
    (xy -38.421521 18.301609) (xy -38.580999 18.052008) (xy -38.718344 17.832198) (xy -38.841964 17.626963) (xy -38.960268 17.421086)
    (xy -39.081662 17.199352) (xy -39.214555 16.946546) (xy -39.367356 16.647451) (xy -39.548471 16.286851) (xy -39.674451 16.034194)
    (xy -39.835569 15.709761) (xy -39.982 15.413403) (xy -40.108549 15.155757) (xy -40.210017 14.947461) (xy -40.281207 14.799153)
    (xy -40.316923 14.721472) (xy -40.320114 14.712619) (xy -40.338752 14.66027) (xy -40.387821 14.545489) (xy -40.457051 14.392223)
    (xy -40.463347 14.378597) (xy -40.534311 14.218322) (xy -40.585544 14.089341) (xy -40.606514 14.01828) (xy -40.60658 14.016535)
    (xy -40.627866 13.932893) (xy -40.651769 13.881024) (xy -40.714322 13.744733) (xy -40.798371 13.529634) (xy -40.899749 13.248896)
    (xy -41.014293 12.915687) (xy -41.137838 12.543177) (xy -41.266219 12.144534) (xy -41.395271 11.732927) (xy -41.520831 11.321524)
    (xy -41.638733 10.923494) (xy -41.744813 10.552007) (xy -41.834906 10.22023) (xy -41.904848 9.941333) (xy -41.923672 9.85921)
    (xy -42.037715 9.334108) (xy -42.137875 8.845938) (xy -42.226724 8.378139) (xy -42.306831 7.914152) (xy -42.380767 7.437416)
    (xy -42.451104 6.931371) (xy -42.520412 6.379457) (xy -42.591263 5.765114) (xy -42.664855 5.084774) (xy -42.686114 4.823236)
    (xy -42.704216 4.480449) (xy -42.719107 4.0706) (xy -42.73073 3.607879) (xy -42.739031 3.106475) (xy -42.743955 2.580576)
    (xy -42.745446 2.04437) (xy -42.743449 1.512047) (xy -42.737909 0.997795) (xy -42.728771 0.515802) (xy -42.71598 0.080258)
    (xy -42.699479 -0.294648) (xy -42.686579 -0.501316) (xy -42.640677 -1.073023) (xy -42.584504 -1.672099) (xy -42.520166 -2.281538)
    (xy -42.449767 -2.884333) (xy -42.375411 -3.463477) (xy -42.299202 -4.001964) (xy -42.223245 -4.482785) (xy -42.149644 -4.888935)
    (xy -42.134218 -4.965414) (xy -42.103709 -5.116356) (xy -42.061815 -5.327557) (xy -42.01516 -5.5655) (xy -41.987968 -5.705452)
    (xy -41.917812 -6.044279) (xy -41.825531 -6.454319) (xy -41.71628 -6.915275) (xy -41.595213 -7.406849) (xy -41.467484 -7.908744)
    (xy -41.338248 -8.400664) (xy -41.212659 -8.862312) (xy -41.095872 -9.27339) (xy -41.00586 -9.572745) (xy -40.875635 -9.984265)
    (xy -40.737268 -10.410441) (xy -40.596657 -10.833923) (xy -40.459699 -11.237361) (xy -40.332291 -11.603405) (xy -40.220331 -11.914706)
    (xy -40.129715 -12.153913) (xy -40.12141 -12.174813) (xy -40.036751 -12.387914) (xy -39.960458 -12.58236) (xy -39.902697 -12.732114)
    (xy -39.879064 -12.795489) (xy -39.826303 -12.932138) (xy -39.758467 -13.095589) (xy -39.739457 -13.139423) (xy -39.689297 -13.264627)
    (xy -39.675665 -13.357741) (xy -39.698101 -13.463504) (xy -39.73506 -13.569122) (xy -39.753269 -13.625205) (xy -39.768569 -13.690911)
    (xy -39.781166 -13.774308) (xy -39.791264 -13.883466) (xy -39.79907 -14.026453) (xy -39.804789 -14.21134) (xy -39.808626 -14.446194)
    (xy -39.810787 -14.739086) (xy -39.811477 -15.098083) (xy -39.810902 -15.531256) (xy -39.809268 -16.046674) (xy -39.807757 -16.424061)
    (xy -39.804035 -17.071941) (xy -39.798671 -17.643839) (xy -39.791734 -18.136704) (xy -39.783291 -18.547488) (xy -39.77341 -18.873139)
    (xy -39.762158 -19.11061) (xy -39.749602 -19.256849) (xy -39.744318 -19.288722) (xy -39.718213 -19.438327) (xy -39.693033 -19.647683)
    (xy -39.668382 -19.92253) (xy -39.643862 -20.268605) (xy -39.619077 -20.691646) (xy -39.593628 -21.197392) (xy -39.567119 -21.791581)
    (xy -39.560948 -21.938534) (xy -39.517786 -22.936258) (xy -39.474743 -23.846347) (xy -39.431257 -24.67665) (xy -39.386765 -25.435019)
    (xy -39.340705 -26.129304) (xy -39.292515 -26.767356) (xy -39.241634 -27.357026) (xy -39.187497 -27.906165) (xy -39.129545 -28.422622)
    (xy -39.067213 -28.914249) (xy -39.054938 -29.0047) (xy -38.977002 -29.565221) (xy -38.908125 -30.04101) (xy -38.846316 -30.442183)
    (xy -38.789584 -30.778853) (xy -38.735935 -31.061137) (xy -38.68338 -31.299149) (xy -38.629926 -31.503005) (xy -38.573581 -31.682819)
    (xy -38.512355 -31.848707) (xy -38.478798 -31.930753) (xy -38.410727 -32.097905) (xy -38.356438 -32.241169) (xy -38.329631 -32.322933)
    (xy -38.295111 -32.403601) (xy -38.222196 -32.542166) (xy -38.1233 -32.715678) (xy -38.059465 -32.822402) (xy -37.863829 -33.111204)
    (xy -37.668211 -33.32915) (xy -37.550941 -33.429208) (xy -37.415344 -33.530626) (xy -37.309089 -33.603989) (xy -37.25452 -33.633899)
    (xy -37.253844 -33.633968) (xy -37.195206 -33.654017) (xy -37.078628 -33.703988) (xy -36.962921 -33.757312) (xy -36.870243 -33.79961)
    (xy -36.786242 -33.830457) (xy -36.694495 -33.851361) (xy -36.578578 -33.863832) (xy -36.422069 -33.86938) (xy -36.208545 -33.869512))
   (stroke (width 0.5) (type solid)) (fill no) (layer "Edge.Cuts")))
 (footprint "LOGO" (layer "F.Cu") (at 131 108)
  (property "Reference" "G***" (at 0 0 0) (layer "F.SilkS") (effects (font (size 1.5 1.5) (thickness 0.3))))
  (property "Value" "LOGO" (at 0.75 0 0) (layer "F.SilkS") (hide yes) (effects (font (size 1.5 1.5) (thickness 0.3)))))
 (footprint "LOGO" (layer "F.Cu") (at 161 78 -10)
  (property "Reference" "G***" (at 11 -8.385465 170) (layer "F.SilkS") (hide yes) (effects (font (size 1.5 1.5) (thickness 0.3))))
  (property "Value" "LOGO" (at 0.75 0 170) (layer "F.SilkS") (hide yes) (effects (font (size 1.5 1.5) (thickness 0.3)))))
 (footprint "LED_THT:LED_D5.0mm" (layer "F.Cu") (at 119.581103 88.75)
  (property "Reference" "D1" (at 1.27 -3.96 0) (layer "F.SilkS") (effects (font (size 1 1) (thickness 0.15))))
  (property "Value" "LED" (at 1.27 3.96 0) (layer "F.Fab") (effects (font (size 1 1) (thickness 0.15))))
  (pad "1" thru_hole rect (at 0 0) (size 1.8 1.8) (drill 0.9) (layers "*.Cu" "*.Mask") (remove_unused_layers no) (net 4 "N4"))
  (pad "2" thru_hole circle (at 2.54 0) (size 1.8 1.8) (drill 0.9) (layers "*.Cu" "*.Mask") (remove_unused_layers no) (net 2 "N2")))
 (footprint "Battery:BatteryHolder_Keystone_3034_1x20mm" (layer "B.Cu") (at 130.581103 94.75)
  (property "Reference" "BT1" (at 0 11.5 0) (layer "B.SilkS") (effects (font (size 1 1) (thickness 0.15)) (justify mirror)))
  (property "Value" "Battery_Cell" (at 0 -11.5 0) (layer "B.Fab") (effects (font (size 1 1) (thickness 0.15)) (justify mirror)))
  (pad "1" smd rect (at -10.985 0) (size 1.27 5.08) (layers "B.Cu" "B.Mask" "B.Paste") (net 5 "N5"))
  (pad "1" smd rect (at 10.985 0) (size 1.27 5.08) (layers "B.Cu" "B.Mask" "B.Paste") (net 5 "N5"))
  (pad "2" smd circle (at 0 0) (size 17.8 17.8) (layers "B.Cu" "B.Mask") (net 3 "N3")))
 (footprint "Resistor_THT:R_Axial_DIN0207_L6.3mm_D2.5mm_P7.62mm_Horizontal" (layer "B.Cu") (at 139.391103 112.75 180)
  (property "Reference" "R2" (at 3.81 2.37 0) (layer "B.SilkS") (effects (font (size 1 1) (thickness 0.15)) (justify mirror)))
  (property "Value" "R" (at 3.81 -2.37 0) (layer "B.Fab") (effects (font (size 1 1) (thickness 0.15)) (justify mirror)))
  (pad "1" thru_hole circle (at 0 0 180) (size 1.6 1.6) (drill 0.8) (layers "*.Cu" "*.Mask") (remove_unused_layers no) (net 5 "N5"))
  (pad "2" thru_hole circle (at 7.62 0 180) (size 1.6 1.6) (drill 0.8) (layers "*.Cu" "*.Mask") (remove_unused_layers no) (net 1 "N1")))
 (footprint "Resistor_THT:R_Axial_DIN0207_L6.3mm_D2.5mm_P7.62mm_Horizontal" (layer "B.Cu") (at 129.391103 112.75 180)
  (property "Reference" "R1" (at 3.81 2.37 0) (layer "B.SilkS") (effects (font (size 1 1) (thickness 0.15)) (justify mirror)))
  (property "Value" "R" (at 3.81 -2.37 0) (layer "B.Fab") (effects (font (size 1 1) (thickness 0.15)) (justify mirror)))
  (pad "1" thru_hole circle (at 0 0 180) (size 1.6 1.6) (drill 0.8) (layers "*.Cu" "*.Mask") (remove_unused_layers no) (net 5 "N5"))
  (pad "2" thru_hole circle (at 7.62 0 180) (size 1.6 1.6) (drill 0.8) (layers "*.Cu" "*.Mask") (remove_unused_layers no) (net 4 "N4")))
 (via (at 131 77) (size 5.5) (drill 5) (layers "F.Cu" "B.Cu") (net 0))
 (segment (start 138.290103 113.851) (end 139.391103 112.75) (width 0.2) (layer "F.Cu") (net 5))
 (segment (start 129.391103 112.75) (end 130.492103 113.851) (width 0.2) (layer "F.Cu") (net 5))
 (segment (start 130.492103 113.851) (end 138.290103 113.851) (width 0.2) (layer "F.Cu") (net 5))
 (segment (start 123.328153 112.75) (end 129.391103 112.75) (width 0.2) (layer "B.Cu") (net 5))
 (segment (start 141.566103 110.575) (end 139.391103 112.75) (width 0.2) (layer "B.Cu") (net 5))
 (segment (start 119.596103 109.01795) (end 123.328153 112.75) (width 0.2) (layer "B.Cu") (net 5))
 (segment (start 141.566103 94.75) (end 141.566103 110.575) (width 0.2) (layer "B.Cu") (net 5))
 (segment (start 119.596103 94.75) (end 119.596103 109.01795) (width 0.2) (layer "B.Cu") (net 5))
 (segment (start 130.581103 94.75) (end 130.581103 101.25) (width 0.2) (layer "B.Cu") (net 3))
 (segment (start 130.581103 94.75) (end 130.581103 100.75) (width 0.2) (layer "B.Cu") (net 3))
 (segment (start 130.581103 101.25) (end 133.581103 104.25) (width 0.2) (layer "B.Cu") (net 3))
 (segment (start 130.581103 100.75) (end 127.081103 104.25) (width 0.2) (layer "B.Cu") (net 3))
 (segment (start 127.081103 99.75) (end 127.081103 93.71) (width 0.2) (layer "F.Cu") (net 2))
 (segment (start 127.081103 93.71) (end 122.121103 88.75) (width 0.2) (layer "F.Cu") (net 2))
 (segment (start 140.380103 87.549) (end 123.322103 87.549) (width 0.2) (layer "F.Cu") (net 2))
 (segment (start 141.581103 88.75) (end 140.380103 87.549) (width 0.2) (layer "F.Cu") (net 2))
 (segment (start 123.322103 87.549) (end 122.121103 88.75) (width 0.2) (layer "F.Cu") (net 2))
 (segment (start 127.081103 99.75) (end 133.581103 99.75) (width 0.2) (layer "F.Cu") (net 2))
 (segment (start 119.581103 89.75) (end 121.771103 91.94) (width 0.2) (layer "F.Cu") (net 4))
 (segment (start 121.771103 91.94) (end 121.771103 112.75) (width 0.2) (layer "F.Cu") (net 4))
 (segment (start 119.581103 88.75) (end 119.581103 89.75) (width 0.2) (layer "F.Cu") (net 4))
 (segment (start 139.041103 105.48) (end 131.771103 112.75) (width 0.2) (layer "F.Cu") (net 1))
 (segment (start 139.041103 88.75) (end 139.041103 105.48) (width 0.2) (layer "F.Cu") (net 1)))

